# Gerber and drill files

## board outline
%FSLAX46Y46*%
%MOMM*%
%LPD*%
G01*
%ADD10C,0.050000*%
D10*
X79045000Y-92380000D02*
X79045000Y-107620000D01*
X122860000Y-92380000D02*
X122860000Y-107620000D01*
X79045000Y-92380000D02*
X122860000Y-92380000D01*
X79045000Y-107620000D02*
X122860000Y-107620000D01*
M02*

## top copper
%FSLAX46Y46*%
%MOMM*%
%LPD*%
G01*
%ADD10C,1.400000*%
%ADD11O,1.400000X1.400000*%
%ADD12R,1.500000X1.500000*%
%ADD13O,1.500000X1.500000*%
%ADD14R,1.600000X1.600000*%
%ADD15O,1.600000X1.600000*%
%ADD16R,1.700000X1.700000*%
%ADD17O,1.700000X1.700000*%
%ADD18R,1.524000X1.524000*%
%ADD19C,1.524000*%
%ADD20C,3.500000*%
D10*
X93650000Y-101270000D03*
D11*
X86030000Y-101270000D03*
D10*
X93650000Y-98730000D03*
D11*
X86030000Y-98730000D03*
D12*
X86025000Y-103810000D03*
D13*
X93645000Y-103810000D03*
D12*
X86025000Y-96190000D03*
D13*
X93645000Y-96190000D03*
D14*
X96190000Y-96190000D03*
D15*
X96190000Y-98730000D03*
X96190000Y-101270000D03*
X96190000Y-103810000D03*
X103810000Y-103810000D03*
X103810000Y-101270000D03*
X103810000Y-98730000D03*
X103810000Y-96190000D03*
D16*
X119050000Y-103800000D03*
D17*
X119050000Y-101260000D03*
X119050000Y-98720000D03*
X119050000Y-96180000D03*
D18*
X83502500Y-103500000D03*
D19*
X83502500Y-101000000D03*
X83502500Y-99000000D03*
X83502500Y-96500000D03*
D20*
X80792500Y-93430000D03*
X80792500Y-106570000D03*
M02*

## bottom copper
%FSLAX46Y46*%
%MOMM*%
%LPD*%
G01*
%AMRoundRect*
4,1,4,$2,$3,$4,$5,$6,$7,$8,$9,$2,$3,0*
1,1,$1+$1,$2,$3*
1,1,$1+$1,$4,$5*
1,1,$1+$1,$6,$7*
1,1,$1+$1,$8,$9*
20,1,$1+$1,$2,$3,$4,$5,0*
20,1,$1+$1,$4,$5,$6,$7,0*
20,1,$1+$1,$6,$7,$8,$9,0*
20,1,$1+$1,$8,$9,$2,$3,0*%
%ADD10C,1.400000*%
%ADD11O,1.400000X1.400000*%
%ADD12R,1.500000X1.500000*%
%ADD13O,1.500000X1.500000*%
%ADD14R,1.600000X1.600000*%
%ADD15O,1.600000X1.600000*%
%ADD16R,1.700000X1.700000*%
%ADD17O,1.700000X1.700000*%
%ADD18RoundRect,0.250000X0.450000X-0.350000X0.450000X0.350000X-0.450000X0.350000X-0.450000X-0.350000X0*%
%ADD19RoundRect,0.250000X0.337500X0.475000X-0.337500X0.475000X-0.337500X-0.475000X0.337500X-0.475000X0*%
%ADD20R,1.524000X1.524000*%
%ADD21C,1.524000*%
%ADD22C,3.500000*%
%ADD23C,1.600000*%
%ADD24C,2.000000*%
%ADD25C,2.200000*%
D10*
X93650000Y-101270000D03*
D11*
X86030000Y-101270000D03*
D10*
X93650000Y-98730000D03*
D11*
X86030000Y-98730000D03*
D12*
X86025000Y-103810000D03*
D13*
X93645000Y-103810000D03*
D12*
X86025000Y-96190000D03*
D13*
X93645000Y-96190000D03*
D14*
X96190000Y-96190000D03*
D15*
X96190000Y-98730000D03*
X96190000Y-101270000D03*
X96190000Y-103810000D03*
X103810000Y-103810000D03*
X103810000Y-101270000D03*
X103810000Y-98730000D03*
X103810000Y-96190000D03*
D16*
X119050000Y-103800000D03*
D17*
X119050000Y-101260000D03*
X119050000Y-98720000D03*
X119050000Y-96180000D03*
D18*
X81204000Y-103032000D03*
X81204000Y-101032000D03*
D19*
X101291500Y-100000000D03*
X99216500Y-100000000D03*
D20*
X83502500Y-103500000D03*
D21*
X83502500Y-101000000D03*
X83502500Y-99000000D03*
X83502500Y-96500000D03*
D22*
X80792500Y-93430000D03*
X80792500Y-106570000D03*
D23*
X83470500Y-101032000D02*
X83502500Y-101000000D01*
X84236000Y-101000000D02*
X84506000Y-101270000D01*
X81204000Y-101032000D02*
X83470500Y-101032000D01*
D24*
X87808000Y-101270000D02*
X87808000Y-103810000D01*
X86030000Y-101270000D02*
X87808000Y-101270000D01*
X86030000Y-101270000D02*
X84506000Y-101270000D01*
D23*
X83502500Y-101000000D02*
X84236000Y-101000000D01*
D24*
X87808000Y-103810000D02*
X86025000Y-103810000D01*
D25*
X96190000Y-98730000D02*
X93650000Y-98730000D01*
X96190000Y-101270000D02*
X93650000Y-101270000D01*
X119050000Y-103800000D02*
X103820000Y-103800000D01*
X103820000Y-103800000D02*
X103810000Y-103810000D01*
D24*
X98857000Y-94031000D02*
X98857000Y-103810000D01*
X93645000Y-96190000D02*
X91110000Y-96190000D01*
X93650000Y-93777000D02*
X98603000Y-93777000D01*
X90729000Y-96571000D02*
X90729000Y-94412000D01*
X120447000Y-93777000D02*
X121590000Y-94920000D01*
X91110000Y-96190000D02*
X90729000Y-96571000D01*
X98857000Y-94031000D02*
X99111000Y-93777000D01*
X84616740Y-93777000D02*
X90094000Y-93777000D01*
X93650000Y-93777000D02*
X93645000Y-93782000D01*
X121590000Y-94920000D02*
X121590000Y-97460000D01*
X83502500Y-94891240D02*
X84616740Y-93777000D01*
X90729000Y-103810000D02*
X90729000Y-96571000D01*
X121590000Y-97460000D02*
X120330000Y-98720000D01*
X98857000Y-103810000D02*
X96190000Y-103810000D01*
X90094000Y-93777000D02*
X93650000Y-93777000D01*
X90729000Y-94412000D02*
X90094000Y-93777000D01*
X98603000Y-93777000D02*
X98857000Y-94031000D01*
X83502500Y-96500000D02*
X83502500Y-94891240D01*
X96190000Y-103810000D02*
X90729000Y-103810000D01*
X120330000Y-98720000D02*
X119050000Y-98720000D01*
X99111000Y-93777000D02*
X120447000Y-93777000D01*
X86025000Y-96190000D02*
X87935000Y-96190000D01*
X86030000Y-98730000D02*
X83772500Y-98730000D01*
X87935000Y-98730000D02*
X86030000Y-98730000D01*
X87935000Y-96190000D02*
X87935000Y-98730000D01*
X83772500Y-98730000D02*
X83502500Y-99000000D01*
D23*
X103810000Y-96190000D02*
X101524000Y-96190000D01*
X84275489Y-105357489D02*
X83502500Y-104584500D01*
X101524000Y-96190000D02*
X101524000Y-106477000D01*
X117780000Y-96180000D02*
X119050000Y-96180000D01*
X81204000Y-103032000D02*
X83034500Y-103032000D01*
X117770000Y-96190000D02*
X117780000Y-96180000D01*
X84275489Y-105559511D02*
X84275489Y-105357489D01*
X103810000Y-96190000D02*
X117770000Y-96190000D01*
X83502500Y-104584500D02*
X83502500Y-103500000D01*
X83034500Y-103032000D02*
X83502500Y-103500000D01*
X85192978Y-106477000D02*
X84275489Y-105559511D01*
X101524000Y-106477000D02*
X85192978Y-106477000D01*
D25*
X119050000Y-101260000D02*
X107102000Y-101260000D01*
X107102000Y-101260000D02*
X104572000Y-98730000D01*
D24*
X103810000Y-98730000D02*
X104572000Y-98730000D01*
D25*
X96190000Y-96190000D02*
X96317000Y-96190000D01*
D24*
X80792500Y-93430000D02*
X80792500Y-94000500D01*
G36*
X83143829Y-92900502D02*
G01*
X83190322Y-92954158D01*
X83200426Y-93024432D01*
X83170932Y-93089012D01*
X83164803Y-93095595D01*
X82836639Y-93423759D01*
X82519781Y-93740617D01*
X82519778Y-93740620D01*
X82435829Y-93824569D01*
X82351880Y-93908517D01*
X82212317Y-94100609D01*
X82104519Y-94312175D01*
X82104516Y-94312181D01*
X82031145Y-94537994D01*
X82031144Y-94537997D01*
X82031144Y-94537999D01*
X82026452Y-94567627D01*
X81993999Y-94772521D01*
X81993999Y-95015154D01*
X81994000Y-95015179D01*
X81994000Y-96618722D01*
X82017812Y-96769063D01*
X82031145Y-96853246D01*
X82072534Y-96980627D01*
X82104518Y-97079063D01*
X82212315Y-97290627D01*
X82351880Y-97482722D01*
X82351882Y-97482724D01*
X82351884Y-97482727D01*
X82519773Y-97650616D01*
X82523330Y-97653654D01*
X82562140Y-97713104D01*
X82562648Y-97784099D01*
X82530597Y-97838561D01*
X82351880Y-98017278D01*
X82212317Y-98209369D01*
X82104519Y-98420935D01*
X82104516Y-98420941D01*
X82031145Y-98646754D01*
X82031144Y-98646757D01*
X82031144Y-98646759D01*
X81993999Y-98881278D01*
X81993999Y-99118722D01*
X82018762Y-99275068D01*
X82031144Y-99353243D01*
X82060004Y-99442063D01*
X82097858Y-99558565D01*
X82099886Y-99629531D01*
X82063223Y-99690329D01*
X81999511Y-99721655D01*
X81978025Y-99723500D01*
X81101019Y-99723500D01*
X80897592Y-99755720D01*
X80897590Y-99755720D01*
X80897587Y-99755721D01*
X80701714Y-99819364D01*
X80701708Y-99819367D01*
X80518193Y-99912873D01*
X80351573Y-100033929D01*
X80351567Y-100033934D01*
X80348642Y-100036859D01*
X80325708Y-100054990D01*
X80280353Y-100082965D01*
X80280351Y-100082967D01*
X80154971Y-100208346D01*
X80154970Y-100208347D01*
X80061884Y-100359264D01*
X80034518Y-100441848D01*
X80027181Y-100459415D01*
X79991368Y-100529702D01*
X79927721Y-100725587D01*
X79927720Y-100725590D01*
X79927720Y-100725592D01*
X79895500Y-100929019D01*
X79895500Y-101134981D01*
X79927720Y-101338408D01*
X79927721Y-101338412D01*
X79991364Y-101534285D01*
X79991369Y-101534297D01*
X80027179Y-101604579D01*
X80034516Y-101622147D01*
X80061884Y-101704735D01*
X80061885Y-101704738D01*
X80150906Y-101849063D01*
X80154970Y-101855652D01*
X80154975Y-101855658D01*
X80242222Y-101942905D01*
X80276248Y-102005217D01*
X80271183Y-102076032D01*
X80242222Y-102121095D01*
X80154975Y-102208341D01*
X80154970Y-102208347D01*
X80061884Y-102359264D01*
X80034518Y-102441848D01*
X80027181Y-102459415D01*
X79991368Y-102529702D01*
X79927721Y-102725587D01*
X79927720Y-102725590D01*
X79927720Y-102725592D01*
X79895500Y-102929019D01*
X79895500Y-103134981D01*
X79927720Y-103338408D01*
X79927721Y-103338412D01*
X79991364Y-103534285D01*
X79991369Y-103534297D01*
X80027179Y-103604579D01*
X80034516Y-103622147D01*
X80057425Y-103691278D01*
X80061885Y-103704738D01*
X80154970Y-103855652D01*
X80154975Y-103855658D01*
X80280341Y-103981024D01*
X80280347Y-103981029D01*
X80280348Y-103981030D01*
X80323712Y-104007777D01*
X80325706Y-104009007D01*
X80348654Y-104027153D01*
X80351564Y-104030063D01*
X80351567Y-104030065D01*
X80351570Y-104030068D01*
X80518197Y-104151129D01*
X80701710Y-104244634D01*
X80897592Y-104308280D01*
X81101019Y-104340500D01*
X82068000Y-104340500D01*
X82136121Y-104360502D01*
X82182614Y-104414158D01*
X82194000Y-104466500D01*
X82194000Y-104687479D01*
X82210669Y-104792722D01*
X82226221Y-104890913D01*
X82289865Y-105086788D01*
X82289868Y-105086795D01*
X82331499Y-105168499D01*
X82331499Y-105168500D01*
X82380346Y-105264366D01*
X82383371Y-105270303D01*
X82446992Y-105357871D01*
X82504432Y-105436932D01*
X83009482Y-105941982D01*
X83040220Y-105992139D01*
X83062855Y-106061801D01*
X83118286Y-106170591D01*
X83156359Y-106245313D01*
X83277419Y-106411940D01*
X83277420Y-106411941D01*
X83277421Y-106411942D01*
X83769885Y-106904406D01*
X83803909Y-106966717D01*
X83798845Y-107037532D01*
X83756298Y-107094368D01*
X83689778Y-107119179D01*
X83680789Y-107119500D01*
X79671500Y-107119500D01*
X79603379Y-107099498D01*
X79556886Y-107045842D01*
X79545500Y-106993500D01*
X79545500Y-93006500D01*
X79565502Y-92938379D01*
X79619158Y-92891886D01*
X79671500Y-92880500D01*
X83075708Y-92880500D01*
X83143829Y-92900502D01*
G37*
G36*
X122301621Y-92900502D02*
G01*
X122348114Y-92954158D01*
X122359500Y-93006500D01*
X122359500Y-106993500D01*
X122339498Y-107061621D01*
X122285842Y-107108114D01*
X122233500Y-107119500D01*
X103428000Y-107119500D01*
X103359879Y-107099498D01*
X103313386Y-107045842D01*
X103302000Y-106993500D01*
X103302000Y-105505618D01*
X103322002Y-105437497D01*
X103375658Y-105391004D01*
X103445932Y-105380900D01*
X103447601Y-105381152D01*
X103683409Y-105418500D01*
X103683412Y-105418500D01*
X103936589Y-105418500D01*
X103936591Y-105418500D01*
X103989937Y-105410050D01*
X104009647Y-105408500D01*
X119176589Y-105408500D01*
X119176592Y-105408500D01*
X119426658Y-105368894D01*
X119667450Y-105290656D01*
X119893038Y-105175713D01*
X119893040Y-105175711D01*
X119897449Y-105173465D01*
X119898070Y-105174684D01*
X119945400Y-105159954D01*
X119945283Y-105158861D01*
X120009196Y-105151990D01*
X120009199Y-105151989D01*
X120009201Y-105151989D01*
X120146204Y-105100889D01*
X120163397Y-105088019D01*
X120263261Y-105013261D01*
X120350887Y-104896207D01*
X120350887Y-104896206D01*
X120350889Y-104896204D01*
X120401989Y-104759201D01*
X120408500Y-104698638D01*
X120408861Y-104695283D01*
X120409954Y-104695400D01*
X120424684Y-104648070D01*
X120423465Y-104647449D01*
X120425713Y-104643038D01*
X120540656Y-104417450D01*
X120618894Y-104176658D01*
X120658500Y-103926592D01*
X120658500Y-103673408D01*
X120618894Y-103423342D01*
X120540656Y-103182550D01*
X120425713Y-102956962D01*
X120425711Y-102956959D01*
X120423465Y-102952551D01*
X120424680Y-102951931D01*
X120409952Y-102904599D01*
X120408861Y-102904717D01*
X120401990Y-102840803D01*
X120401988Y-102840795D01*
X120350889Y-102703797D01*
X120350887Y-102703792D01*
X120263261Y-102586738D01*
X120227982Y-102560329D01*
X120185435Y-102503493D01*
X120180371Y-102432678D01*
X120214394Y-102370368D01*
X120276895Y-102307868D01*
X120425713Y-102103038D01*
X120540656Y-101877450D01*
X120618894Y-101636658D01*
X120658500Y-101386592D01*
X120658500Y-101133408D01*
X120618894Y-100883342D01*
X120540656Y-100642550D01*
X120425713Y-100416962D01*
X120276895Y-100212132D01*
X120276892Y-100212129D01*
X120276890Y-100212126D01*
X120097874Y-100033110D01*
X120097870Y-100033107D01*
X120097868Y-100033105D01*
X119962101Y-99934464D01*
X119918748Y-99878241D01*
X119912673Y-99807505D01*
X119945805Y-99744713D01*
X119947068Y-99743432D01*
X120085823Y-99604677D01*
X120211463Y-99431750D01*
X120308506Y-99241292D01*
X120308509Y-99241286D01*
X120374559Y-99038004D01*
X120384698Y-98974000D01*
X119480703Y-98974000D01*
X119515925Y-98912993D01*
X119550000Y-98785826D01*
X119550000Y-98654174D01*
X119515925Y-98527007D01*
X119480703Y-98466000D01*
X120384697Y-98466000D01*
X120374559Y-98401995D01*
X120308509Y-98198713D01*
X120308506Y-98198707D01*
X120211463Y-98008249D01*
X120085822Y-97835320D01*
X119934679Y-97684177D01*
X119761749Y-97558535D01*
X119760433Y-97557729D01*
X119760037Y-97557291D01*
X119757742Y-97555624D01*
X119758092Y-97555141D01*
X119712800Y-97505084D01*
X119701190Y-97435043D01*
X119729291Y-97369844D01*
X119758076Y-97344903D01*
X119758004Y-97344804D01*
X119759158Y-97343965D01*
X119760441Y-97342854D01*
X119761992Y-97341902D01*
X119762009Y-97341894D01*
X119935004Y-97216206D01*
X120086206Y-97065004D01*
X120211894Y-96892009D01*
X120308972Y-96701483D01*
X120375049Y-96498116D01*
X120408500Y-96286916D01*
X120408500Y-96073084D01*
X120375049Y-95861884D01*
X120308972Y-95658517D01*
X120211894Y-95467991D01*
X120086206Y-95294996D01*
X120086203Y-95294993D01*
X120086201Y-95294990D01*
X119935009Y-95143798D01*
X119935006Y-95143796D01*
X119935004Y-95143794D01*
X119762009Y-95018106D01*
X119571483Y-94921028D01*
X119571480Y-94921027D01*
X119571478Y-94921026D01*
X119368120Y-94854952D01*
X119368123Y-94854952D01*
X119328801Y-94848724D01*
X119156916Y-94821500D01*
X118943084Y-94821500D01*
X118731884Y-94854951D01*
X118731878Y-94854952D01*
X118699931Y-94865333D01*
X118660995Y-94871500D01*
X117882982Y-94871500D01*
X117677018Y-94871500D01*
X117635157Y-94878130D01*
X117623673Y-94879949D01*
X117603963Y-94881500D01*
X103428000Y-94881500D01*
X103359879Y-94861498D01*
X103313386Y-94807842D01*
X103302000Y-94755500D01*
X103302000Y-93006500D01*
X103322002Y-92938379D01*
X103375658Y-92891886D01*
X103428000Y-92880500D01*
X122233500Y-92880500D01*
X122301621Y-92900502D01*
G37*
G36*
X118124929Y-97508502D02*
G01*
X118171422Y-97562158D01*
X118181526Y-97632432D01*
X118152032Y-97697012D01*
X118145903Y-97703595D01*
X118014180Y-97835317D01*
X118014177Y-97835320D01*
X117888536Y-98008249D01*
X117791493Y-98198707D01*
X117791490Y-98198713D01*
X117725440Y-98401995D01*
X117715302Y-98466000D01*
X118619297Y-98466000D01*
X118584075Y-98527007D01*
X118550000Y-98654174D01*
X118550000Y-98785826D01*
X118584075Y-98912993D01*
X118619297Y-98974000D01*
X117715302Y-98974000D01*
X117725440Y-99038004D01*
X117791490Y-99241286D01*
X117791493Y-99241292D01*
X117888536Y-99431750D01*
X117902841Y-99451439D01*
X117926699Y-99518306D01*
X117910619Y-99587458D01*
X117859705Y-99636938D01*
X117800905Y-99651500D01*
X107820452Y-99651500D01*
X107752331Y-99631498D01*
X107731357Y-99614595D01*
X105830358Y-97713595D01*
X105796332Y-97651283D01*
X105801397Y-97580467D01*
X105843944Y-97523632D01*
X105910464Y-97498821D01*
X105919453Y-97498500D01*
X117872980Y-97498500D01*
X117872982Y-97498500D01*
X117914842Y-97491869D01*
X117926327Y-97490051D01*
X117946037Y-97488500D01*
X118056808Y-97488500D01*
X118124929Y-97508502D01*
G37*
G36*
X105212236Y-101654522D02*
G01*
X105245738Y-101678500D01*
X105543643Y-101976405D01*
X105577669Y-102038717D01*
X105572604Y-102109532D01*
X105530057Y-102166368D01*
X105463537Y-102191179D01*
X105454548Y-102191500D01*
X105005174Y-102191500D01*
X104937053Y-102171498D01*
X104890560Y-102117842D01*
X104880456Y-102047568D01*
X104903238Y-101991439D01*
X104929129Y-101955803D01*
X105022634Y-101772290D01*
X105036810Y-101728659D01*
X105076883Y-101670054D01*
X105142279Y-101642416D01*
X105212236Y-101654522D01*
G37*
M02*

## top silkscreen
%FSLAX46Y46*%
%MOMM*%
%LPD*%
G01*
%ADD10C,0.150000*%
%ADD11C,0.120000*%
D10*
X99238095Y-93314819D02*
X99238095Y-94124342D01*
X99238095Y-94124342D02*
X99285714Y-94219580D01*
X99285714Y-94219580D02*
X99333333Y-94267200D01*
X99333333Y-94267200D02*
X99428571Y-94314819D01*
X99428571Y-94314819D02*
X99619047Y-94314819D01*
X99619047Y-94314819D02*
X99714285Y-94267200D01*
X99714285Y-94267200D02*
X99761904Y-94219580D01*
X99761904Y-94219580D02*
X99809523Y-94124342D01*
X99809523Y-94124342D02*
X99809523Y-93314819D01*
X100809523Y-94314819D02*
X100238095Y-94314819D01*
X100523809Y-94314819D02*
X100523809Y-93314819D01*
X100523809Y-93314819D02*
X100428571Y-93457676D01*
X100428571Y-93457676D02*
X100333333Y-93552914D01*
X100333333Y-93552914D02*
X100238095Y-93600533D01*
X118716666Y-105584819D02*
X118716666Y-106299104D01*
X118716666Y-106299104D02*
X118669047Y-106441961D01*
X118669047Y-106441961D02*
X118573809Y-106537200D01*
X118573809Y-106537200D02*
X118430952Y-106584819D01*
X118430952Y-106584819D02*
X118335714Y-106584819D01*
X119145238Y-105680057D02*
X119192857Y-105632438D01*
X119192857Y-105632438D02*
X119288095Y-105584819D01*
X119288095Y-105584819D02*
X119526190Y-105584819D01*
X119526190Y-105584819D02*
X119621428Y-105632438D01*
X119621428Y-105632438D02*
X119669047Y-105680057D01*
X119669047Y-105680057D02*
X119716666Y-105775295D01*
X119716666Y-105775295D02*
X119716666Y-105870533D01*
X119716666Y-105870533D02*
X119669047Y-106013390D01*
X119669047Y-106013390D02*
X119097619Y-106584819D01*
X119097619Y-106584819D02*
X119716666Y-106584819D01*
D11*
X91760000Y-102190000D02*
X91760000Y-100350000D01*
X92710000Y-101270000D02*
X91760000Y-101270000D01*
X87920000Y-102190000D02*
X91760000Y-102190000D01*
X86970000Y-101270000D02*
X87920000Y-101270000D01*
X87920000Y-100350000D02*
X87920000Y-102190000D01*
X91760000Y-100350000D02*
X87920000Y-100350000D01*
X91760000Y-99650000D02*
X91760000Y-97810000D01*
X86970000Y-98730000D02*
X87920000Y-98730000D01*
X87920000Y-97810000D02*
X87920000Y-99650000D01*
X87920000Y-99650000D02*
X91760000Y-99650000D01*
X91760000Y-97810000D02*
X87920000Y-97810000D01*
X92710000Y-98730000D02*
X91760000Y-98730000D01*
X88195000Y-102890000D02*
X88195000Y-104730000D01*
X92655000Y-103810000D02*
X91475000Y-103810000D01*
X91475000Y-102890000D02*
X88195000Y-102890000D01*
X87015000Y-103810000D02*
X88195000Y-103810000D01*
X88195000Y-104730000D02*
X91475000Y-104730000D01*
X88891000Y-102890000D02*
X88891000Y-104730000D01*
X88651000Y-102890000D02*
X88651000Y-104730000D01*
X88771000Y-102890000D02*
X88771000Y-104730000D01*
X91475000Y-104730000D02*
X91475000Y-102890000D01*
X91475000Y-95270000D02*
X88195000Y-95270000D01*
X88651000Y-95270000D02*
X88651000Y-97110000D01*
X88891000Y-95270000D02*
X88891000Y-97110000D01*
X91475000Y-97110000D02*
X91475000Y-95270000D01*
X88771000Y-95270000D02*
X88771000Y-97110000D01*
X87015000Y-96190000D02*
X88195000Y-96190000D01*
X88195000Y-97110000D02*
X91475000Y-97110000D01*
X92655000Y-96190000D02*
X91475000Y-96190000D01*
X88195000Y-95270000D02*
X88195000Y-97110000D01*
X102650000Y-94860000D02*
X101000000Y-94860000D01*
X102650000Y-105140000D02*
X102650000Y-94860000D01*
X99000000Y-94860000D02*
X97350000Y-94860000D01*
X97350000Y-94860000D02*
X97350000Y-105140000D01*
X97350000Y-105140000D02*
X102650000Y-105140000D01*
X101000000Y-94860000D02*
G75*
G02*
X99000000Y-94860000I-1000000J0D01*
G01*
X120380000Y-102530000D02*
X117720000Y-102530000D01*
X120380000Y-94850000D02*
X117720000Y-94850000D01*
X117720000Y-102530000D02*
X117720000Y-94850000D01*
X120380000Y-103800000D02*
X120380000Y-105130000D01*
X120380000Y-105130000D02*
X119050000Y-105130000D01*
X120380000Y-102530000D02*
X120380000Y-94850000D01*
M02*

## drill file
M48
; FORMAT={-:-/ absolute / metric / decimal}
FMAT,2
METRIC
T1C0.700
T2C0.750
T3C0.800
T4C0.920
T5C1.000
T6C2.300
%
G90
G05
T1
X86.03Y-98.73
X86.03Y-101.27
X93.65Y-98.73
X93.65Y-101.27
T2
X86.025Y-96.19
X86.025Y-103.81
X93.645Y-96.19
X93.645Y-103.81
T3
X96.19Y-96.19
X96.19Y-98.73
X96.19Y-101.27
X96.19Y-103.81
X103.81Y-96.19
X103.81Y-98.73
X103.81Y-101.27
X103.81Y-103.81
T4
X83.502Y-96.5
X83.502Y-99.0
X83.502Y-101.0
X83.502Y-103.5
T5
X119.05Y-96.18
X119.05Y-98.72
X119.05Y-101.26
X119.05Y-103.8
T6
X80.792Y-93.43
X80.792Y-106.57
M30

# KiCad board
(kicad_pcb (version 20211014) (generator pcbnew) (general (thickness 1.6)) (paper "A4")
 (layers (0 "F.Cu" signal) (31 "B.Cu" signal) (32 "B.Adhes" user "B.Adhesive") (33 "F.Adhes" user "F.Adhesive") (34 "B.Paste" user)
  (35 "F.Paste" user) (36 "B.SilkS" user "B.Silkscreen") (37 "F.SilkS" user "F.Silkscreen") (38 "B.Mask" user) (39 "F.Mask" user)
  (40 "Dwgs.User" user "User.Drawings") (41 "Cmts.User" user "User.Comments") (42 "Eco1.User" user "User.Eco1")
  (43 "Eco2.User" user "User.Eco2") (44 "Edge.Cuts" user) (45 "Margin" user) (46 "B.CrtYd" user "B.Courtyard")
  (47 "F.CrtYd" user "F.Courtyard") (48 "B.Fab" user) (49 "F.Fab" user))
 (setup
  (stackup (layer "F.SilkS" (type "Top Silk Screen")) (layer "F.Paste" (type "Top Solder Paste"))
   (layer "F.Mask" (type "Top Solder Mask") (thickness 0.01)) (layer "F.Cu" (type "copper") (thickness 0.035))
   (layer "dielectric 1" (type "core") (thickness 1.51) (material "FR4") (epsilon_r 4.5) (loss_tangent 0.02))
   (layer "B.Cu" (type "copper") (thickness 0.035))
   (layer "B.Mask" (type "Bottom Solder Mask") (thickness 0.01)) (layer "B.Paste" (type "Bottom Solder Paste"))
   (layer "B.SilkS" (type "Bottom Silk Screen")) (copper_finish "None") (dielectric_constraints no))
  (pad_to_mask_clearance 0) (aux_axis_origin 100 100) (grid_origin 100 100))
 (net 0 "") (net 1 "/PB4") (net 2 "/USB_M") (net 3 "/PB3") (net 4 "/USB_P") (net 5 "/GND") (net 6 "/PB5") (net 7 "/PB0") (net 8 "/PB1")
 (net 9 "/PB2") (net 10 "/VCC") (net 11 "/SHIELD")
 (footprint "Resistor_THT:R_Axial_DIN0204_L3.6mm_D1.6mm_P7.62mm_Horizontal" (layer "F.Cu") (at 93.65 101.27 180)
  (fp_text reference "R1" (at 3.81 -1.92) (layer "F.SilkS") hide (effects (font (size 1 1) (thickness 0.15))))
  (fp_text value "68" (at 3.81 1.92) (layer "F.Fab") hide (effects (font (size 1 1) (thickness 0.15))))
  (fp_line (start 1.89 -0.92) (end 1.89 0.92) (layer "F.SilkS") (width 0.12))
  (fp_line (start 0.94 0) (end 1.89 0) (layer "F.SilkS") (width 0.12))
  (fp_line (start 5.73 -0.92) (end 1.89 -0.92) (layer "F.SilkS") (width 0.12))
  (fp_line (start 6.68 0) (end 5.73 0) (layer "F.SilkS") (width 0.12))
  (fp_line (start 5.73 0.92) (end 5.73 -0.92) (layer "F.SilkS") (width 0.12))
  (fp_line (start 1.89 0.92) (end 5.73 0.92) (layer "F.SilkS") (width 0.12))
  (pad "1" thru_hole circle locked (at 0 0 180) (size 1.4 1.4) (drill 0.7) (layers *.Cu *.Mask) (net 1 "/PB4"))
  (pad "2" thru_hole oval locked (at 7.62 0 180) (size 1.4 1.4) (drill 0.7) (layers *.Cu *.Mask) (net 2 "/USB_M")))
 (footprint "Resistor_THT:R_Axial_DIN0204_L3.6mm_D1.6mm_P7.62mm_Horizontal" (layer "F.Cu") (at 93.65 98.73 180)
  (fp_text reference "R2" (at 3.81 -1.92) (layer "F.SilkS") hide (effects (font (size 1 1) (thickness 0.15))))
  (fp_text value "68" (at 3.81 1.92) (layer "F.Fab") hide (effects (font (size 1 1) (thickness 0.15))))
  (fp_line (start 1.89 -0.92) (end 1.89 0.92) (layer "F.SilkS") (width 0.12))
  (fp_line (start 6.68 0) (end 5.73 0) (layer "F.SilkS") (width 0.12))
  (fp_line (start 5.73 0.92) (end 5.73 -0.92) (layer "F.SilkS") (width 0.12))
  (fp_line (start 5.73 -0.92) (end 1.89 -0.92) (layer "F.SilkS") (width 0.12))
  (fp_line (start 1.89 0.92) (end 5.73 0.92) (layer "F.SilkS") (width 0.12))
  (fp_line (start 0.94 0) (end 1.89 0) (layer "F.SilkS") (width 0.12))
  (pad "1" thru_hole circle locked (at 0 0 180) (size 1.4 1.4) (drill 0.7) (layers *.Cu *.Mask) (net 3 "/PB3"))
  (pad "2" thru_hole oval locked (at 7.62 0 180) (size 1.4 1.4) (drill 0.7) (layers *.Cu *.Mask) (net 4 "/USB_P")))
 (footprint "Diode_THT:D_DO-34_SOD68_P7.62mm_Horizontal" (layer "F.Cu") (at 86.025 103.81)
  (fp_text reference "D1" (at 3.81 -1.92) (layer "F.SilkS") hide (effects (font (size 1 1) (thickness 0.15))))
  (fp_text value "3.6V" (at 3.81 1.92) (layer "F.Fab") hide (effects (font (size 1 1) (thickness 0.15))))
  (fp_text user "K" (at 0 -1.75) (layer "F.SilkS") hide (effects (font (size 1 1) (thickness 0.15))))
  (fp_line (start 2.17 -0.92) (end 2.17 0.92) (layer "F.SilkS") (width 0.12))
  (fp_line (start 6.63 0) (end 5.45 0) (layer "F.SilkS") (width 0.12))
  (fp_line (start 5.45 -0.92) (end 2.17 -0.92) (layer "F.SilkS") (width 0.12))
  (fp_line (start 0.99 0) (end 2.17 0) (layer "F.SilkS") (width 0.12))
  (fp_line (start 2.17 0.92) (end 5.45 0.92) (layer "F.SilkS") (width 0.12))
  (fp_line (start 2.866 -0.92) (end 2.866 0.92) (layer "F.SilkS") (width 0.12))
  (fp_line (start 2.626 -0.92) (end 2.626 0.92) (layer "F.SilkS") (width 0.12))
  (fp_line (start 2.746 -0.92) (end 2.746 0.92) (layer "F.SilkS") (width 0.12))
  (fp_line (start 5.45 0.92) (end 5.45 -0.92) (layer "F.SilkS") (width 0.12))
  (pad "1" thru_hole rect locked (at 0 0) (size 1.5 1.5) (drill 0.75) (layers *.Cu *.Mask) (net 2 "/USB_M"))
  (pad "2" thru_hole oval locked (at 7.62 0) (size 1.5 1.5) (drill 0.75) (layers *.Cu *.Mask) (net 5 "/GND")))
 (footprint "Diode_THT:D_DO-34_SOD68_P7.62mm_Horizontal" (layer "F.Cu") (at 86.025 96.19)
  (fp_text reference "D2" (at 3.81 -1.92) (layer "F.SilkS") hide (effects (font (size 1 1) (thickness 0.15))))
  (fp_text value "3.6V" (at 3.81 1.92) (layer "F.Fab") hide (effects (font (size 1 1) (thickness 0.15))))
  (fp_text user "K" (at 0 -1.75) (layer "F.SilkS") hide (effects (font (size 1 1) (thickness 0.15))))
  (fp_line (start 5.45 -0.92) (end 2.17 -0.92) (layer "F.SilkS") (width 0.12))
  (fp_line (start 2.626 -0.92) (end 2.626 0.92) (layer "F.SilkS") (width 0.12))
  (fp_line (start 2.866 -0.92) (end 2.866 0.92) (layer "F.SilkS") (width 0.12))
  (fp_line (start 5.45 0.92) (end 5.45 -0.92) (layer "F.SilkS") (width 0.12))
  (fp_line (start 2.746 -0.92) (end 2.746 0.92) (layer "F.SilkS") (width 0.12))
  (fp_line (start 0.99 0) (end 2.17 0) (layer "F.SilkS") (width 0.12))
  (fp_line (start 2.17 0.92) (end 5.45 0.92) (layer "F.SilkS") (width 0.12))
  (fp_line (start 6.63 0) (end 5.45 0) (layer "F.SilkS") (width 0.12))
  (fp_line (start 2.17 -0.92) (end 2.17 0.92) (layer "F.SilkS") (width 0.12))
  (pad "1" thru_hole rect locked (at 0 0) (size 1.5 1.5) (drill 0.75) (layers *.Cu *.Mask) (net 4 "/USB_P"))
  (pad "2" thru_hole oval locked (at 7.62 0) (size 1.5 1.5) (drill 0.75) (layers *.Cu *.Mask) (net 5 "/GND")))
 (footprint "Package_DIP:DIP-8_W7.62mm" (layer "F.Cu") (at 96.19 96.19)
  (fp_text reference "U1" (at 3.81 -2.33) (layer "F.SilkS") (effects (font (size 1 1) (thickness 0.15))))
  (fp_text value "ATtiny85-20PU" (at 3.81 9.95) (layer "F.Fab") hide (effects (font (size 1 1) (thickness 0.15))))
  (fp_line (start 6.46 -1.33) (end 4.81 -1.33) (layer "F.SilkS") (width 0.12))
  (fp_line (start 6.46 8.95) (end 6.46 -1.33) (layer "F.SilkS") (width 0.12))
  (fp_line (start 2.81 -1.33) (end 1.16 -1.33) (layer "F.SilkS") (width 0.12))
  (fp_line (start 1.16 -1.33) (end 1.16 8.95) (layer "F.SilkS") (width 0.12))
  (fp_line (start 1.16 8.95) (end 6.46 8.95) (layer "F.SilkS") (width 0.12))
  (fp_arc (start 4.81 -1.33) (mid 3.81 -0.33) (end 2.81 -1.33) (layer "F.SilkS") (width 0.12))
  (pad "1" thru_hole rect locked (at 0 0) (size 1.6 1.6) (drill 0.8) (layers *.Cu *.Mask) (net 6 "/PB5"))
  (pad "2" thru_hole oval locked (at 0 2.54) (size 1.6 1.6) (drill 0.8) (layers *.Cu *.Mask) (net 3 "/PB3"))
  (pad "3" thru_hole oval locked (at 0 5.08) (size 1.6 1.6) (drill 0.8) (layers *.Cu *.Mask) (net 1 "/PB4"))
  (pad "4" thru_hole oval locked (at 0 7.62) (size 1.6 1.6) (drill 0.8) (layers *.Cu *.Mask) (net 5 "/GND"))
  (pad "5" thru_hole oval locked (at 7.62 7.62) (size 1.6 1.6) (drill 0.8) (layers *.Cu *.Mask) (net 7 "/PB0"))
  (pad "6" thru_hole oval locked (at 7.62 5.08) (size 1.6 1.6) (drill 0.8) (layers *.Cu *.Mask) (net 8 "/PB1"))
  (pad "7" thru_hole oval locked (at 7.62 2.54) (size 1.6 1.6) (drill 0.8) (layers *.Cu *.Mask) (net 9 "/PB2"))
  (pad "8" thru_hole oval locked (at 7.62 0) (size 1.6 1.6) (drill 0.8) (layers *.Cu *.Mask) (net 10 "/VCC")))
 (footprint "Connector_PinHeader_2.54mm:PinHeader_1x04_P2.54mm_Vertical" (layer "F.Cu") (at 119.05 103.8 180)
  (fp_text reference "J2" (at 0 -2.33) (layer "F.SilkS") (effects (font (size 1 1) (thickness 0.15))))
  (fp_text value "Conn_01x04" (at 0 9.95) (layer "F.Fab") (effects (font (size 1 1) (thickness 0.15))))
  (fp_line (start -1.33 1.27) (end 1.33 1.27) (layer "F.SilkS") (width 0.12))
  (fp_line (start -1.33 8.95) (end 1.33 8.95) (layer "F.SilkS") (width 0.12))
  (fp_line (start 1.33 1.27) (end 1.33 8.95) (layer "F.SilkS") (width 0.12))
  (fp_line (start -1.33 0) (end -1.33 -1.33) (layer "F.SilkS") (width 0.12))
  (fp_line (start -1.33 -1.33) (end 0 -1.33) (layer "F.SilkS") (width 0.12))
  (fp_line (start -1.33 1.27) (end -1.33 8.95) (layer "F.SilkS") (width 0.12))
  (pad "1" thru_hole rect (at 0 0 180) (size 1.7 1.7) (drill 1) (layers *.Cu *.Mask) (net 7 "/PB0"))
  (pad "2" thru_hole oval (at 0 2.54 180) (size 1.7 1.7) (drill 1) (layers *.Cu *.Mask) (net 9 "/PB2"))
  (pad "3" thru_hole oval (at 0 5.08 180) (size 1.7 1.7) (drill 1) (layers *.Cu *.Mask) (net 5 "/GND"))
  (pad "4" thru_hole oval (at 0 7.62 180) (size 1.7 1.7) (drill 1) (layers *.Cu *.Mask) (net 10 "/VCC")))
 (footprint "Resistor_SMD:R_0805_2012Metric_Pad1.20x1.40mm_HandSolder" (layer "B.Cu") (at 81.204 102.032 90)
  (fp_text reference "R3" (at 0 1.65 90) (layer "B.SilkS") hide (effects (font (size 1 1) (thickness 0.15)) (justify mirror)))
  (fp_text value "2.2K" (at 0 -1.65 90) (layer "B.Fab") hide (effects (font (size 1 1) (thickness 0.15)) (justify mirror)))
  (pad "1" smd roundrect locked (at -1 0 90) (size 1.2 1.4) (layers "B.Cu" "B.Paste" "B.Mask") (roundrect_rratio 0.2083333333)
   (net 10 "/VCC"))
  (pad "2" smd roundrect locked (at 1 0 90) (size 1.2 1.4) (layers "B.Cu" "B.Paste" "B.Mask") (roundrect_rratio 0.2083333333)
   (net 2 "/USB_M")))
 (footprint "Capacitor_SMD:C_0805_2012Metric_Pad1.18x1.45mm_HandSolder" (layer "B.Cu") (at 100.254 100 180)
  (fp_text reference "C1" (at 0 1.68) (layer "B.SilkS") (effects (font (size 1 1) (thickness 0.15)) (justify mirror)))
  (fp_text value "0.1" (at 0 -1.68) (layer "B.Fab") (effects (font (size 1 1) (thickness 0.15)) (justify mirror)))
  (pad "1" smd roundrect locked (at -1.0375 0 180) (size 1.175 1.45) (layers "B.Cu" "B.Paste" "B.Mask") (roundrect_rratio 0.2127659574)
   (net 10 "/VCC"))
  (pad "2" smd roundrect locked (at 1.0375 0 180) (size 1.175 1.45) (layers "B.Cu" "B.Paste" "B.Mask") (roundrect_rratio 0.2127659574)
   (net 5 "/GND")))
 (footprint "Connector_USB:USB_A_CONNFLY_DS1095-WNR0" (layer "B.Cu") (at 83.5025 103.5 90)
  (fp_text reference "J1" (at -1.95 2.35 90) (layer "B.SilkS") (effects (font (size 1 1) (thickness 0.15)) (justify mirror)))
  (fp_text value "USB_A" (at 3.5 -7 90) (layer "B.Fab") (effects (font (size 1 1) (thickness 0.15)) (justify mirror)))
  (pad "1" thru_hole rect (at 0 0 90) (size 1.524 1.524) (drill 0.92) (layers *.Cu *.Mask) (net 10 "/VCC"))
  (pad "2" thru_hole circle (at 2.5 0 90) (size 1.524 1.524) (drill 0.92) (layers *.Cu *.Mask) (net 2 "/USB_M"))
  (pad "3" thru_hole circle (at 4.5 0 90) (size 1.524 1.524) (drill 0.92) (layers *.Cu *.Mask) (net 4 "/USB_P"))
  (pad "4" thru_hole circle (at 7 0 90) (size 1.524 1.524) (drill 0.92) (layers *.Cu *.Mask) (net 5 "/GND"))
  (pad "5" thru_hole circle (at 10.07 -2.71 90) (size 3.5 3.5) (drill 2.3) (layers *.Cu *.Mask) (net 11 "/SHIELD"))
  (pad "5" thru_hole circle (at -3.07 -2.71 90) (size 3.5 3.5) (drill 2.3) (layers *.Cu *.Mask) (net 11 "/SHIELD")))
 (gr_line (start 79.045 92.38) (end 79.045 107.62) (layer "Edge.Cuts") (width 0.05))
 (gr_line (start 122.86 92.38) (end 122.86 107.62) (layer "Edge.Cuts") (width 0.05))
 (gr_line (start 79.045 92.38) (end 122.86 92.38) (layer "Edge.Cuts") (width 0.05))
 (gr_line (start 79.045 107.62) (end 122.86 107.62) (layer "Edge.Cuts") (width 0.05))
 (segment (start 83.4705 101.032) (end 83.5025 101) (width 1.6) (layer "B.Cu") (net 2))
 (segment (start 84.236 101) (end 84.506 101.27) (width 1.6) (layer "B.Cu") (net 2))
 (segment (start 81.204 101.032) (end 83.4705 101.032) (width 1.6) (layer "B.Cu") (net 2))
 (segment (start 87.808 101.27) (end 87.808 103.81) (width 2) (layer "B.Cu") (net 2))
 (segment (start 86.03 101.27) (end 87.808 101.27) (width 2) (layer "B.Cu") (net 2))
 (segment (start 86.03 101.27) (end 84.506 101.27) (width 2) (layer "B.Cu") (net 2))
 (segment (start 83.5025 101) (end 84.236 101) (width 1.6) (layer "B.Cu") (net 2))
 (segment (start 87.808 103.81) (end 86.025 103.81) (width 2) (layer "B.Cu") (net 2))
 (segment (start 96.19 98.73) (end 93.65 98.73) (width 2.2) (layer "B.Cu") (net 3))
 (segment (start 96.19 101.27) (end 93.65 101.27) (width 2.2) (layer "B.Cu") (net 1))
 (segment (start 119.05 103.8) (end 103.82 103.8) (width 2.2) (layer "B.Cu") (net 7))
 (segment (start 103.82 103.8) (end 103.81 103.81) (width 2.2) (layer "B.Cu") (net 7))
 (segment (start 98.857 94.031) (end 98.857 103.81) (width 2) (layer "B.Cu") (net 5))
 (segment (start 93.645 96.19) (end 91.11 96.19) (width 2) (layer "B.Cu") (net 5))
 (segment (start 93.65 93.777) (end 98.603 93.777) (width 2) (layer "B.Cu") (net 5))
 (segment (start 90.729 96.571) (end 90.729 94.412) (width 2) (layer "B.Cu") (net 5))
 (segment (start 120.447 93.777) (end 121.59 94.92) (width 2) (layer "B.Cu") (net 5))
 (segment (start 91.11 96.19) (end 90.729 96.571) (width 2) (layer "B.Cu") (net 5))
 (segment (start 98.857 94.031) (end 99.111 93.777) (width 2) (layer "B.Cu") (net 5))
 (segment (start 84.61674 93.777) (end 90.094 93.777) (width 2) (layer "B.Cu") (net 5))
 (segment (start 93.65 93.777) (end 93.645 93.782) (width 2) (layer "B.Cu") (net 5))
 (segment (start 121.59 94.92) (end 121.59 97.46) (width 2) (layer "B.Cu") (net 5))
 (segment (start 83.5025 94.89124) (end 84.61674 93.777) (width 2) (layer "B.Cu") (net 5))
 (segment (start 90.729 103.81) (end 90.729 96.571) (width 2) (layer "B.Cu") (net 5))
 (segment (start 121.59 97.46) (end 120.33 98.72) (width 2) (layer "B.Cu") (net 5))
 (segment (start 98.857 103.81) (end 96.19 103.81) (width 2) (layer "B.Cu") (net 5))
 (segment (start 90.094 93.777) (end 93.65 93.777) (width 2) (layer "B.Cu") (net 5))
 (segment (start 90.729 94.412) (end 90.094 93.777) (width 2) (layer "B.Cu") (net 5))
 (segment (start 98.603 93.777) (end 98.857 94.031) (width 2) (layer "B.Cu") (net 5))
 (segment (start 83.5025 96.5) (end 83.5025 94.89124) (width 2) (layer "B.Cu") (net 5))
 (segment (start 96.19 103.81) (end 90.729 103.81) (width 2) (layer "B.Cu") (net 5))
 (segment (start 120.33 98.72) (end 119.05 98.72) (width 2) (layer "B.Cu") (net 5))
 (segment (start 99.111 93.777) (end 120.447 93.777) (width 2) (layer "B.Cu") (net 5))
 (segment (start 86.025 96.19) (end 87.935 96.19) (width 2) (layer "B.Cu") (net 4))
 (segment (start 86.03 98.73) (end 83.7725 98.73) (width 2) (layer "B.Cu") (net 4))
 (segment (start 87.935 98.73) (end 86.03 98.73) (width 2) (layer "B.Cu") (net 4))
 (segment (start 87.935 96.19) (end 87.935 98.73) (width 2) (layer "B.Cu") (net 4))
 (segment (start 83.7725 98.73) (end 83.5025 99) (width 2) (layer "B.Cu") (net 4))
 (segment (start 103.81 96.19) (end 101.524 96.19) (width 1.6) (layer "B.Cu") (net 10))
 (segment (start 84.275489 105.357489) (end 83.5025 104.5845) (width 1.6) (layer "B.Cu") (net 10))
 (segment (start 101.524 96.19) (end 101.524 106.477) (width 1.6) (layer "B.Cu") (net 10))
 (segment (start 117.78 96.18) (end 119.05 96.18) (width 1.6) (layer "B.Cu") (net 10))
 (segment (start 81.204 103.032) (end 83.0345 103.032) (width 1.6) (layer "B.Cu") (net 10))
 (segment (start 117.77 96.19) (end 117.78 96.18) (width 1.6) (layer "B.Cu") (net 10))
 (segment (start 84.275489 105.559511) (end 84.275489 105.357489) (width 1.6) (layer "B.Cu") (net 10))
 (segment (start 103.81 96.19) (end 117.77 96.19) (width 1.6) (layer "B.Cu") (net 10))
 (segment (start 83.5025 104.5845) (end 83.5025 103.5) (width 1.6) (layer "B.Cu") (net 10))
 (segment (start 83.0345 103.032) (end 83.5025 103.5) (width 1.6) (layer "B.Cu") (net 10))
 (segment (start 85.192978 106.477) (end 84.275489 105.559511) (width 1.6) (layer "B.Cu") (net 10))
 (segment (start 101.524 106.477) (end 85.192978 106.477) (width 1.6) (layer "B.Cu") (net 10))
 (segment (start 119.05 101.26) (end 107.102 101.26) (width 2.2) (layer "B.Cu") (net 9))
 (segment (start 107.102 101.26) (end 104.572 98.73) (width 2.2) (layer "B.Cu") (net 9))
 (segment (start 103.81 98.73) (end 104.572 98.73) (width 2) (layer "B.Cu") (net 9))
 (segment (start 96.19 96.19) (end 96.317 96.19) (width 2.2) (layer "B.Cu") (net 6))
 (segment (start 80.7925 93.43) (end 80.7925 94.0005) (width 2) (layer "B.Cu") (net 11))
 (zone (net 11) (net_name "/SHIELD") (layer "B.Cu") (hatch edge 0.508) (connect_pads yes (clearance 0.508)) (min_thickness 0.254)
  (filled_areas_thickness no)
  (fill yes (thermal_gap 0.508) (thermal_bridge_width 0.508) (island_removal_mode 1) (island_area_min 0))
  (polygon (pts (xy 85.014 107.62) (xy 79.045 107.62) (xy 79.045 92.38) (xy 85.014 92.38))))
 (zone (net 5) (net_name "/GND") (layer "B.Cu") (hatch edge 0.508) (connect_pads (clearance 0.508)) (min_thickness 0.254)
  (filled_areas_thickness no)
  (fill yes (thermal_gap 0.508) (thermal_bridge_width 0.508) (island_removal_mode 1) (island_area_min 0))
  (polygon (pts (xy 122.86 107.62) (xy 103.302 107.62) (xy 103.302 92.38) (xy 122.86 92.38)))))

